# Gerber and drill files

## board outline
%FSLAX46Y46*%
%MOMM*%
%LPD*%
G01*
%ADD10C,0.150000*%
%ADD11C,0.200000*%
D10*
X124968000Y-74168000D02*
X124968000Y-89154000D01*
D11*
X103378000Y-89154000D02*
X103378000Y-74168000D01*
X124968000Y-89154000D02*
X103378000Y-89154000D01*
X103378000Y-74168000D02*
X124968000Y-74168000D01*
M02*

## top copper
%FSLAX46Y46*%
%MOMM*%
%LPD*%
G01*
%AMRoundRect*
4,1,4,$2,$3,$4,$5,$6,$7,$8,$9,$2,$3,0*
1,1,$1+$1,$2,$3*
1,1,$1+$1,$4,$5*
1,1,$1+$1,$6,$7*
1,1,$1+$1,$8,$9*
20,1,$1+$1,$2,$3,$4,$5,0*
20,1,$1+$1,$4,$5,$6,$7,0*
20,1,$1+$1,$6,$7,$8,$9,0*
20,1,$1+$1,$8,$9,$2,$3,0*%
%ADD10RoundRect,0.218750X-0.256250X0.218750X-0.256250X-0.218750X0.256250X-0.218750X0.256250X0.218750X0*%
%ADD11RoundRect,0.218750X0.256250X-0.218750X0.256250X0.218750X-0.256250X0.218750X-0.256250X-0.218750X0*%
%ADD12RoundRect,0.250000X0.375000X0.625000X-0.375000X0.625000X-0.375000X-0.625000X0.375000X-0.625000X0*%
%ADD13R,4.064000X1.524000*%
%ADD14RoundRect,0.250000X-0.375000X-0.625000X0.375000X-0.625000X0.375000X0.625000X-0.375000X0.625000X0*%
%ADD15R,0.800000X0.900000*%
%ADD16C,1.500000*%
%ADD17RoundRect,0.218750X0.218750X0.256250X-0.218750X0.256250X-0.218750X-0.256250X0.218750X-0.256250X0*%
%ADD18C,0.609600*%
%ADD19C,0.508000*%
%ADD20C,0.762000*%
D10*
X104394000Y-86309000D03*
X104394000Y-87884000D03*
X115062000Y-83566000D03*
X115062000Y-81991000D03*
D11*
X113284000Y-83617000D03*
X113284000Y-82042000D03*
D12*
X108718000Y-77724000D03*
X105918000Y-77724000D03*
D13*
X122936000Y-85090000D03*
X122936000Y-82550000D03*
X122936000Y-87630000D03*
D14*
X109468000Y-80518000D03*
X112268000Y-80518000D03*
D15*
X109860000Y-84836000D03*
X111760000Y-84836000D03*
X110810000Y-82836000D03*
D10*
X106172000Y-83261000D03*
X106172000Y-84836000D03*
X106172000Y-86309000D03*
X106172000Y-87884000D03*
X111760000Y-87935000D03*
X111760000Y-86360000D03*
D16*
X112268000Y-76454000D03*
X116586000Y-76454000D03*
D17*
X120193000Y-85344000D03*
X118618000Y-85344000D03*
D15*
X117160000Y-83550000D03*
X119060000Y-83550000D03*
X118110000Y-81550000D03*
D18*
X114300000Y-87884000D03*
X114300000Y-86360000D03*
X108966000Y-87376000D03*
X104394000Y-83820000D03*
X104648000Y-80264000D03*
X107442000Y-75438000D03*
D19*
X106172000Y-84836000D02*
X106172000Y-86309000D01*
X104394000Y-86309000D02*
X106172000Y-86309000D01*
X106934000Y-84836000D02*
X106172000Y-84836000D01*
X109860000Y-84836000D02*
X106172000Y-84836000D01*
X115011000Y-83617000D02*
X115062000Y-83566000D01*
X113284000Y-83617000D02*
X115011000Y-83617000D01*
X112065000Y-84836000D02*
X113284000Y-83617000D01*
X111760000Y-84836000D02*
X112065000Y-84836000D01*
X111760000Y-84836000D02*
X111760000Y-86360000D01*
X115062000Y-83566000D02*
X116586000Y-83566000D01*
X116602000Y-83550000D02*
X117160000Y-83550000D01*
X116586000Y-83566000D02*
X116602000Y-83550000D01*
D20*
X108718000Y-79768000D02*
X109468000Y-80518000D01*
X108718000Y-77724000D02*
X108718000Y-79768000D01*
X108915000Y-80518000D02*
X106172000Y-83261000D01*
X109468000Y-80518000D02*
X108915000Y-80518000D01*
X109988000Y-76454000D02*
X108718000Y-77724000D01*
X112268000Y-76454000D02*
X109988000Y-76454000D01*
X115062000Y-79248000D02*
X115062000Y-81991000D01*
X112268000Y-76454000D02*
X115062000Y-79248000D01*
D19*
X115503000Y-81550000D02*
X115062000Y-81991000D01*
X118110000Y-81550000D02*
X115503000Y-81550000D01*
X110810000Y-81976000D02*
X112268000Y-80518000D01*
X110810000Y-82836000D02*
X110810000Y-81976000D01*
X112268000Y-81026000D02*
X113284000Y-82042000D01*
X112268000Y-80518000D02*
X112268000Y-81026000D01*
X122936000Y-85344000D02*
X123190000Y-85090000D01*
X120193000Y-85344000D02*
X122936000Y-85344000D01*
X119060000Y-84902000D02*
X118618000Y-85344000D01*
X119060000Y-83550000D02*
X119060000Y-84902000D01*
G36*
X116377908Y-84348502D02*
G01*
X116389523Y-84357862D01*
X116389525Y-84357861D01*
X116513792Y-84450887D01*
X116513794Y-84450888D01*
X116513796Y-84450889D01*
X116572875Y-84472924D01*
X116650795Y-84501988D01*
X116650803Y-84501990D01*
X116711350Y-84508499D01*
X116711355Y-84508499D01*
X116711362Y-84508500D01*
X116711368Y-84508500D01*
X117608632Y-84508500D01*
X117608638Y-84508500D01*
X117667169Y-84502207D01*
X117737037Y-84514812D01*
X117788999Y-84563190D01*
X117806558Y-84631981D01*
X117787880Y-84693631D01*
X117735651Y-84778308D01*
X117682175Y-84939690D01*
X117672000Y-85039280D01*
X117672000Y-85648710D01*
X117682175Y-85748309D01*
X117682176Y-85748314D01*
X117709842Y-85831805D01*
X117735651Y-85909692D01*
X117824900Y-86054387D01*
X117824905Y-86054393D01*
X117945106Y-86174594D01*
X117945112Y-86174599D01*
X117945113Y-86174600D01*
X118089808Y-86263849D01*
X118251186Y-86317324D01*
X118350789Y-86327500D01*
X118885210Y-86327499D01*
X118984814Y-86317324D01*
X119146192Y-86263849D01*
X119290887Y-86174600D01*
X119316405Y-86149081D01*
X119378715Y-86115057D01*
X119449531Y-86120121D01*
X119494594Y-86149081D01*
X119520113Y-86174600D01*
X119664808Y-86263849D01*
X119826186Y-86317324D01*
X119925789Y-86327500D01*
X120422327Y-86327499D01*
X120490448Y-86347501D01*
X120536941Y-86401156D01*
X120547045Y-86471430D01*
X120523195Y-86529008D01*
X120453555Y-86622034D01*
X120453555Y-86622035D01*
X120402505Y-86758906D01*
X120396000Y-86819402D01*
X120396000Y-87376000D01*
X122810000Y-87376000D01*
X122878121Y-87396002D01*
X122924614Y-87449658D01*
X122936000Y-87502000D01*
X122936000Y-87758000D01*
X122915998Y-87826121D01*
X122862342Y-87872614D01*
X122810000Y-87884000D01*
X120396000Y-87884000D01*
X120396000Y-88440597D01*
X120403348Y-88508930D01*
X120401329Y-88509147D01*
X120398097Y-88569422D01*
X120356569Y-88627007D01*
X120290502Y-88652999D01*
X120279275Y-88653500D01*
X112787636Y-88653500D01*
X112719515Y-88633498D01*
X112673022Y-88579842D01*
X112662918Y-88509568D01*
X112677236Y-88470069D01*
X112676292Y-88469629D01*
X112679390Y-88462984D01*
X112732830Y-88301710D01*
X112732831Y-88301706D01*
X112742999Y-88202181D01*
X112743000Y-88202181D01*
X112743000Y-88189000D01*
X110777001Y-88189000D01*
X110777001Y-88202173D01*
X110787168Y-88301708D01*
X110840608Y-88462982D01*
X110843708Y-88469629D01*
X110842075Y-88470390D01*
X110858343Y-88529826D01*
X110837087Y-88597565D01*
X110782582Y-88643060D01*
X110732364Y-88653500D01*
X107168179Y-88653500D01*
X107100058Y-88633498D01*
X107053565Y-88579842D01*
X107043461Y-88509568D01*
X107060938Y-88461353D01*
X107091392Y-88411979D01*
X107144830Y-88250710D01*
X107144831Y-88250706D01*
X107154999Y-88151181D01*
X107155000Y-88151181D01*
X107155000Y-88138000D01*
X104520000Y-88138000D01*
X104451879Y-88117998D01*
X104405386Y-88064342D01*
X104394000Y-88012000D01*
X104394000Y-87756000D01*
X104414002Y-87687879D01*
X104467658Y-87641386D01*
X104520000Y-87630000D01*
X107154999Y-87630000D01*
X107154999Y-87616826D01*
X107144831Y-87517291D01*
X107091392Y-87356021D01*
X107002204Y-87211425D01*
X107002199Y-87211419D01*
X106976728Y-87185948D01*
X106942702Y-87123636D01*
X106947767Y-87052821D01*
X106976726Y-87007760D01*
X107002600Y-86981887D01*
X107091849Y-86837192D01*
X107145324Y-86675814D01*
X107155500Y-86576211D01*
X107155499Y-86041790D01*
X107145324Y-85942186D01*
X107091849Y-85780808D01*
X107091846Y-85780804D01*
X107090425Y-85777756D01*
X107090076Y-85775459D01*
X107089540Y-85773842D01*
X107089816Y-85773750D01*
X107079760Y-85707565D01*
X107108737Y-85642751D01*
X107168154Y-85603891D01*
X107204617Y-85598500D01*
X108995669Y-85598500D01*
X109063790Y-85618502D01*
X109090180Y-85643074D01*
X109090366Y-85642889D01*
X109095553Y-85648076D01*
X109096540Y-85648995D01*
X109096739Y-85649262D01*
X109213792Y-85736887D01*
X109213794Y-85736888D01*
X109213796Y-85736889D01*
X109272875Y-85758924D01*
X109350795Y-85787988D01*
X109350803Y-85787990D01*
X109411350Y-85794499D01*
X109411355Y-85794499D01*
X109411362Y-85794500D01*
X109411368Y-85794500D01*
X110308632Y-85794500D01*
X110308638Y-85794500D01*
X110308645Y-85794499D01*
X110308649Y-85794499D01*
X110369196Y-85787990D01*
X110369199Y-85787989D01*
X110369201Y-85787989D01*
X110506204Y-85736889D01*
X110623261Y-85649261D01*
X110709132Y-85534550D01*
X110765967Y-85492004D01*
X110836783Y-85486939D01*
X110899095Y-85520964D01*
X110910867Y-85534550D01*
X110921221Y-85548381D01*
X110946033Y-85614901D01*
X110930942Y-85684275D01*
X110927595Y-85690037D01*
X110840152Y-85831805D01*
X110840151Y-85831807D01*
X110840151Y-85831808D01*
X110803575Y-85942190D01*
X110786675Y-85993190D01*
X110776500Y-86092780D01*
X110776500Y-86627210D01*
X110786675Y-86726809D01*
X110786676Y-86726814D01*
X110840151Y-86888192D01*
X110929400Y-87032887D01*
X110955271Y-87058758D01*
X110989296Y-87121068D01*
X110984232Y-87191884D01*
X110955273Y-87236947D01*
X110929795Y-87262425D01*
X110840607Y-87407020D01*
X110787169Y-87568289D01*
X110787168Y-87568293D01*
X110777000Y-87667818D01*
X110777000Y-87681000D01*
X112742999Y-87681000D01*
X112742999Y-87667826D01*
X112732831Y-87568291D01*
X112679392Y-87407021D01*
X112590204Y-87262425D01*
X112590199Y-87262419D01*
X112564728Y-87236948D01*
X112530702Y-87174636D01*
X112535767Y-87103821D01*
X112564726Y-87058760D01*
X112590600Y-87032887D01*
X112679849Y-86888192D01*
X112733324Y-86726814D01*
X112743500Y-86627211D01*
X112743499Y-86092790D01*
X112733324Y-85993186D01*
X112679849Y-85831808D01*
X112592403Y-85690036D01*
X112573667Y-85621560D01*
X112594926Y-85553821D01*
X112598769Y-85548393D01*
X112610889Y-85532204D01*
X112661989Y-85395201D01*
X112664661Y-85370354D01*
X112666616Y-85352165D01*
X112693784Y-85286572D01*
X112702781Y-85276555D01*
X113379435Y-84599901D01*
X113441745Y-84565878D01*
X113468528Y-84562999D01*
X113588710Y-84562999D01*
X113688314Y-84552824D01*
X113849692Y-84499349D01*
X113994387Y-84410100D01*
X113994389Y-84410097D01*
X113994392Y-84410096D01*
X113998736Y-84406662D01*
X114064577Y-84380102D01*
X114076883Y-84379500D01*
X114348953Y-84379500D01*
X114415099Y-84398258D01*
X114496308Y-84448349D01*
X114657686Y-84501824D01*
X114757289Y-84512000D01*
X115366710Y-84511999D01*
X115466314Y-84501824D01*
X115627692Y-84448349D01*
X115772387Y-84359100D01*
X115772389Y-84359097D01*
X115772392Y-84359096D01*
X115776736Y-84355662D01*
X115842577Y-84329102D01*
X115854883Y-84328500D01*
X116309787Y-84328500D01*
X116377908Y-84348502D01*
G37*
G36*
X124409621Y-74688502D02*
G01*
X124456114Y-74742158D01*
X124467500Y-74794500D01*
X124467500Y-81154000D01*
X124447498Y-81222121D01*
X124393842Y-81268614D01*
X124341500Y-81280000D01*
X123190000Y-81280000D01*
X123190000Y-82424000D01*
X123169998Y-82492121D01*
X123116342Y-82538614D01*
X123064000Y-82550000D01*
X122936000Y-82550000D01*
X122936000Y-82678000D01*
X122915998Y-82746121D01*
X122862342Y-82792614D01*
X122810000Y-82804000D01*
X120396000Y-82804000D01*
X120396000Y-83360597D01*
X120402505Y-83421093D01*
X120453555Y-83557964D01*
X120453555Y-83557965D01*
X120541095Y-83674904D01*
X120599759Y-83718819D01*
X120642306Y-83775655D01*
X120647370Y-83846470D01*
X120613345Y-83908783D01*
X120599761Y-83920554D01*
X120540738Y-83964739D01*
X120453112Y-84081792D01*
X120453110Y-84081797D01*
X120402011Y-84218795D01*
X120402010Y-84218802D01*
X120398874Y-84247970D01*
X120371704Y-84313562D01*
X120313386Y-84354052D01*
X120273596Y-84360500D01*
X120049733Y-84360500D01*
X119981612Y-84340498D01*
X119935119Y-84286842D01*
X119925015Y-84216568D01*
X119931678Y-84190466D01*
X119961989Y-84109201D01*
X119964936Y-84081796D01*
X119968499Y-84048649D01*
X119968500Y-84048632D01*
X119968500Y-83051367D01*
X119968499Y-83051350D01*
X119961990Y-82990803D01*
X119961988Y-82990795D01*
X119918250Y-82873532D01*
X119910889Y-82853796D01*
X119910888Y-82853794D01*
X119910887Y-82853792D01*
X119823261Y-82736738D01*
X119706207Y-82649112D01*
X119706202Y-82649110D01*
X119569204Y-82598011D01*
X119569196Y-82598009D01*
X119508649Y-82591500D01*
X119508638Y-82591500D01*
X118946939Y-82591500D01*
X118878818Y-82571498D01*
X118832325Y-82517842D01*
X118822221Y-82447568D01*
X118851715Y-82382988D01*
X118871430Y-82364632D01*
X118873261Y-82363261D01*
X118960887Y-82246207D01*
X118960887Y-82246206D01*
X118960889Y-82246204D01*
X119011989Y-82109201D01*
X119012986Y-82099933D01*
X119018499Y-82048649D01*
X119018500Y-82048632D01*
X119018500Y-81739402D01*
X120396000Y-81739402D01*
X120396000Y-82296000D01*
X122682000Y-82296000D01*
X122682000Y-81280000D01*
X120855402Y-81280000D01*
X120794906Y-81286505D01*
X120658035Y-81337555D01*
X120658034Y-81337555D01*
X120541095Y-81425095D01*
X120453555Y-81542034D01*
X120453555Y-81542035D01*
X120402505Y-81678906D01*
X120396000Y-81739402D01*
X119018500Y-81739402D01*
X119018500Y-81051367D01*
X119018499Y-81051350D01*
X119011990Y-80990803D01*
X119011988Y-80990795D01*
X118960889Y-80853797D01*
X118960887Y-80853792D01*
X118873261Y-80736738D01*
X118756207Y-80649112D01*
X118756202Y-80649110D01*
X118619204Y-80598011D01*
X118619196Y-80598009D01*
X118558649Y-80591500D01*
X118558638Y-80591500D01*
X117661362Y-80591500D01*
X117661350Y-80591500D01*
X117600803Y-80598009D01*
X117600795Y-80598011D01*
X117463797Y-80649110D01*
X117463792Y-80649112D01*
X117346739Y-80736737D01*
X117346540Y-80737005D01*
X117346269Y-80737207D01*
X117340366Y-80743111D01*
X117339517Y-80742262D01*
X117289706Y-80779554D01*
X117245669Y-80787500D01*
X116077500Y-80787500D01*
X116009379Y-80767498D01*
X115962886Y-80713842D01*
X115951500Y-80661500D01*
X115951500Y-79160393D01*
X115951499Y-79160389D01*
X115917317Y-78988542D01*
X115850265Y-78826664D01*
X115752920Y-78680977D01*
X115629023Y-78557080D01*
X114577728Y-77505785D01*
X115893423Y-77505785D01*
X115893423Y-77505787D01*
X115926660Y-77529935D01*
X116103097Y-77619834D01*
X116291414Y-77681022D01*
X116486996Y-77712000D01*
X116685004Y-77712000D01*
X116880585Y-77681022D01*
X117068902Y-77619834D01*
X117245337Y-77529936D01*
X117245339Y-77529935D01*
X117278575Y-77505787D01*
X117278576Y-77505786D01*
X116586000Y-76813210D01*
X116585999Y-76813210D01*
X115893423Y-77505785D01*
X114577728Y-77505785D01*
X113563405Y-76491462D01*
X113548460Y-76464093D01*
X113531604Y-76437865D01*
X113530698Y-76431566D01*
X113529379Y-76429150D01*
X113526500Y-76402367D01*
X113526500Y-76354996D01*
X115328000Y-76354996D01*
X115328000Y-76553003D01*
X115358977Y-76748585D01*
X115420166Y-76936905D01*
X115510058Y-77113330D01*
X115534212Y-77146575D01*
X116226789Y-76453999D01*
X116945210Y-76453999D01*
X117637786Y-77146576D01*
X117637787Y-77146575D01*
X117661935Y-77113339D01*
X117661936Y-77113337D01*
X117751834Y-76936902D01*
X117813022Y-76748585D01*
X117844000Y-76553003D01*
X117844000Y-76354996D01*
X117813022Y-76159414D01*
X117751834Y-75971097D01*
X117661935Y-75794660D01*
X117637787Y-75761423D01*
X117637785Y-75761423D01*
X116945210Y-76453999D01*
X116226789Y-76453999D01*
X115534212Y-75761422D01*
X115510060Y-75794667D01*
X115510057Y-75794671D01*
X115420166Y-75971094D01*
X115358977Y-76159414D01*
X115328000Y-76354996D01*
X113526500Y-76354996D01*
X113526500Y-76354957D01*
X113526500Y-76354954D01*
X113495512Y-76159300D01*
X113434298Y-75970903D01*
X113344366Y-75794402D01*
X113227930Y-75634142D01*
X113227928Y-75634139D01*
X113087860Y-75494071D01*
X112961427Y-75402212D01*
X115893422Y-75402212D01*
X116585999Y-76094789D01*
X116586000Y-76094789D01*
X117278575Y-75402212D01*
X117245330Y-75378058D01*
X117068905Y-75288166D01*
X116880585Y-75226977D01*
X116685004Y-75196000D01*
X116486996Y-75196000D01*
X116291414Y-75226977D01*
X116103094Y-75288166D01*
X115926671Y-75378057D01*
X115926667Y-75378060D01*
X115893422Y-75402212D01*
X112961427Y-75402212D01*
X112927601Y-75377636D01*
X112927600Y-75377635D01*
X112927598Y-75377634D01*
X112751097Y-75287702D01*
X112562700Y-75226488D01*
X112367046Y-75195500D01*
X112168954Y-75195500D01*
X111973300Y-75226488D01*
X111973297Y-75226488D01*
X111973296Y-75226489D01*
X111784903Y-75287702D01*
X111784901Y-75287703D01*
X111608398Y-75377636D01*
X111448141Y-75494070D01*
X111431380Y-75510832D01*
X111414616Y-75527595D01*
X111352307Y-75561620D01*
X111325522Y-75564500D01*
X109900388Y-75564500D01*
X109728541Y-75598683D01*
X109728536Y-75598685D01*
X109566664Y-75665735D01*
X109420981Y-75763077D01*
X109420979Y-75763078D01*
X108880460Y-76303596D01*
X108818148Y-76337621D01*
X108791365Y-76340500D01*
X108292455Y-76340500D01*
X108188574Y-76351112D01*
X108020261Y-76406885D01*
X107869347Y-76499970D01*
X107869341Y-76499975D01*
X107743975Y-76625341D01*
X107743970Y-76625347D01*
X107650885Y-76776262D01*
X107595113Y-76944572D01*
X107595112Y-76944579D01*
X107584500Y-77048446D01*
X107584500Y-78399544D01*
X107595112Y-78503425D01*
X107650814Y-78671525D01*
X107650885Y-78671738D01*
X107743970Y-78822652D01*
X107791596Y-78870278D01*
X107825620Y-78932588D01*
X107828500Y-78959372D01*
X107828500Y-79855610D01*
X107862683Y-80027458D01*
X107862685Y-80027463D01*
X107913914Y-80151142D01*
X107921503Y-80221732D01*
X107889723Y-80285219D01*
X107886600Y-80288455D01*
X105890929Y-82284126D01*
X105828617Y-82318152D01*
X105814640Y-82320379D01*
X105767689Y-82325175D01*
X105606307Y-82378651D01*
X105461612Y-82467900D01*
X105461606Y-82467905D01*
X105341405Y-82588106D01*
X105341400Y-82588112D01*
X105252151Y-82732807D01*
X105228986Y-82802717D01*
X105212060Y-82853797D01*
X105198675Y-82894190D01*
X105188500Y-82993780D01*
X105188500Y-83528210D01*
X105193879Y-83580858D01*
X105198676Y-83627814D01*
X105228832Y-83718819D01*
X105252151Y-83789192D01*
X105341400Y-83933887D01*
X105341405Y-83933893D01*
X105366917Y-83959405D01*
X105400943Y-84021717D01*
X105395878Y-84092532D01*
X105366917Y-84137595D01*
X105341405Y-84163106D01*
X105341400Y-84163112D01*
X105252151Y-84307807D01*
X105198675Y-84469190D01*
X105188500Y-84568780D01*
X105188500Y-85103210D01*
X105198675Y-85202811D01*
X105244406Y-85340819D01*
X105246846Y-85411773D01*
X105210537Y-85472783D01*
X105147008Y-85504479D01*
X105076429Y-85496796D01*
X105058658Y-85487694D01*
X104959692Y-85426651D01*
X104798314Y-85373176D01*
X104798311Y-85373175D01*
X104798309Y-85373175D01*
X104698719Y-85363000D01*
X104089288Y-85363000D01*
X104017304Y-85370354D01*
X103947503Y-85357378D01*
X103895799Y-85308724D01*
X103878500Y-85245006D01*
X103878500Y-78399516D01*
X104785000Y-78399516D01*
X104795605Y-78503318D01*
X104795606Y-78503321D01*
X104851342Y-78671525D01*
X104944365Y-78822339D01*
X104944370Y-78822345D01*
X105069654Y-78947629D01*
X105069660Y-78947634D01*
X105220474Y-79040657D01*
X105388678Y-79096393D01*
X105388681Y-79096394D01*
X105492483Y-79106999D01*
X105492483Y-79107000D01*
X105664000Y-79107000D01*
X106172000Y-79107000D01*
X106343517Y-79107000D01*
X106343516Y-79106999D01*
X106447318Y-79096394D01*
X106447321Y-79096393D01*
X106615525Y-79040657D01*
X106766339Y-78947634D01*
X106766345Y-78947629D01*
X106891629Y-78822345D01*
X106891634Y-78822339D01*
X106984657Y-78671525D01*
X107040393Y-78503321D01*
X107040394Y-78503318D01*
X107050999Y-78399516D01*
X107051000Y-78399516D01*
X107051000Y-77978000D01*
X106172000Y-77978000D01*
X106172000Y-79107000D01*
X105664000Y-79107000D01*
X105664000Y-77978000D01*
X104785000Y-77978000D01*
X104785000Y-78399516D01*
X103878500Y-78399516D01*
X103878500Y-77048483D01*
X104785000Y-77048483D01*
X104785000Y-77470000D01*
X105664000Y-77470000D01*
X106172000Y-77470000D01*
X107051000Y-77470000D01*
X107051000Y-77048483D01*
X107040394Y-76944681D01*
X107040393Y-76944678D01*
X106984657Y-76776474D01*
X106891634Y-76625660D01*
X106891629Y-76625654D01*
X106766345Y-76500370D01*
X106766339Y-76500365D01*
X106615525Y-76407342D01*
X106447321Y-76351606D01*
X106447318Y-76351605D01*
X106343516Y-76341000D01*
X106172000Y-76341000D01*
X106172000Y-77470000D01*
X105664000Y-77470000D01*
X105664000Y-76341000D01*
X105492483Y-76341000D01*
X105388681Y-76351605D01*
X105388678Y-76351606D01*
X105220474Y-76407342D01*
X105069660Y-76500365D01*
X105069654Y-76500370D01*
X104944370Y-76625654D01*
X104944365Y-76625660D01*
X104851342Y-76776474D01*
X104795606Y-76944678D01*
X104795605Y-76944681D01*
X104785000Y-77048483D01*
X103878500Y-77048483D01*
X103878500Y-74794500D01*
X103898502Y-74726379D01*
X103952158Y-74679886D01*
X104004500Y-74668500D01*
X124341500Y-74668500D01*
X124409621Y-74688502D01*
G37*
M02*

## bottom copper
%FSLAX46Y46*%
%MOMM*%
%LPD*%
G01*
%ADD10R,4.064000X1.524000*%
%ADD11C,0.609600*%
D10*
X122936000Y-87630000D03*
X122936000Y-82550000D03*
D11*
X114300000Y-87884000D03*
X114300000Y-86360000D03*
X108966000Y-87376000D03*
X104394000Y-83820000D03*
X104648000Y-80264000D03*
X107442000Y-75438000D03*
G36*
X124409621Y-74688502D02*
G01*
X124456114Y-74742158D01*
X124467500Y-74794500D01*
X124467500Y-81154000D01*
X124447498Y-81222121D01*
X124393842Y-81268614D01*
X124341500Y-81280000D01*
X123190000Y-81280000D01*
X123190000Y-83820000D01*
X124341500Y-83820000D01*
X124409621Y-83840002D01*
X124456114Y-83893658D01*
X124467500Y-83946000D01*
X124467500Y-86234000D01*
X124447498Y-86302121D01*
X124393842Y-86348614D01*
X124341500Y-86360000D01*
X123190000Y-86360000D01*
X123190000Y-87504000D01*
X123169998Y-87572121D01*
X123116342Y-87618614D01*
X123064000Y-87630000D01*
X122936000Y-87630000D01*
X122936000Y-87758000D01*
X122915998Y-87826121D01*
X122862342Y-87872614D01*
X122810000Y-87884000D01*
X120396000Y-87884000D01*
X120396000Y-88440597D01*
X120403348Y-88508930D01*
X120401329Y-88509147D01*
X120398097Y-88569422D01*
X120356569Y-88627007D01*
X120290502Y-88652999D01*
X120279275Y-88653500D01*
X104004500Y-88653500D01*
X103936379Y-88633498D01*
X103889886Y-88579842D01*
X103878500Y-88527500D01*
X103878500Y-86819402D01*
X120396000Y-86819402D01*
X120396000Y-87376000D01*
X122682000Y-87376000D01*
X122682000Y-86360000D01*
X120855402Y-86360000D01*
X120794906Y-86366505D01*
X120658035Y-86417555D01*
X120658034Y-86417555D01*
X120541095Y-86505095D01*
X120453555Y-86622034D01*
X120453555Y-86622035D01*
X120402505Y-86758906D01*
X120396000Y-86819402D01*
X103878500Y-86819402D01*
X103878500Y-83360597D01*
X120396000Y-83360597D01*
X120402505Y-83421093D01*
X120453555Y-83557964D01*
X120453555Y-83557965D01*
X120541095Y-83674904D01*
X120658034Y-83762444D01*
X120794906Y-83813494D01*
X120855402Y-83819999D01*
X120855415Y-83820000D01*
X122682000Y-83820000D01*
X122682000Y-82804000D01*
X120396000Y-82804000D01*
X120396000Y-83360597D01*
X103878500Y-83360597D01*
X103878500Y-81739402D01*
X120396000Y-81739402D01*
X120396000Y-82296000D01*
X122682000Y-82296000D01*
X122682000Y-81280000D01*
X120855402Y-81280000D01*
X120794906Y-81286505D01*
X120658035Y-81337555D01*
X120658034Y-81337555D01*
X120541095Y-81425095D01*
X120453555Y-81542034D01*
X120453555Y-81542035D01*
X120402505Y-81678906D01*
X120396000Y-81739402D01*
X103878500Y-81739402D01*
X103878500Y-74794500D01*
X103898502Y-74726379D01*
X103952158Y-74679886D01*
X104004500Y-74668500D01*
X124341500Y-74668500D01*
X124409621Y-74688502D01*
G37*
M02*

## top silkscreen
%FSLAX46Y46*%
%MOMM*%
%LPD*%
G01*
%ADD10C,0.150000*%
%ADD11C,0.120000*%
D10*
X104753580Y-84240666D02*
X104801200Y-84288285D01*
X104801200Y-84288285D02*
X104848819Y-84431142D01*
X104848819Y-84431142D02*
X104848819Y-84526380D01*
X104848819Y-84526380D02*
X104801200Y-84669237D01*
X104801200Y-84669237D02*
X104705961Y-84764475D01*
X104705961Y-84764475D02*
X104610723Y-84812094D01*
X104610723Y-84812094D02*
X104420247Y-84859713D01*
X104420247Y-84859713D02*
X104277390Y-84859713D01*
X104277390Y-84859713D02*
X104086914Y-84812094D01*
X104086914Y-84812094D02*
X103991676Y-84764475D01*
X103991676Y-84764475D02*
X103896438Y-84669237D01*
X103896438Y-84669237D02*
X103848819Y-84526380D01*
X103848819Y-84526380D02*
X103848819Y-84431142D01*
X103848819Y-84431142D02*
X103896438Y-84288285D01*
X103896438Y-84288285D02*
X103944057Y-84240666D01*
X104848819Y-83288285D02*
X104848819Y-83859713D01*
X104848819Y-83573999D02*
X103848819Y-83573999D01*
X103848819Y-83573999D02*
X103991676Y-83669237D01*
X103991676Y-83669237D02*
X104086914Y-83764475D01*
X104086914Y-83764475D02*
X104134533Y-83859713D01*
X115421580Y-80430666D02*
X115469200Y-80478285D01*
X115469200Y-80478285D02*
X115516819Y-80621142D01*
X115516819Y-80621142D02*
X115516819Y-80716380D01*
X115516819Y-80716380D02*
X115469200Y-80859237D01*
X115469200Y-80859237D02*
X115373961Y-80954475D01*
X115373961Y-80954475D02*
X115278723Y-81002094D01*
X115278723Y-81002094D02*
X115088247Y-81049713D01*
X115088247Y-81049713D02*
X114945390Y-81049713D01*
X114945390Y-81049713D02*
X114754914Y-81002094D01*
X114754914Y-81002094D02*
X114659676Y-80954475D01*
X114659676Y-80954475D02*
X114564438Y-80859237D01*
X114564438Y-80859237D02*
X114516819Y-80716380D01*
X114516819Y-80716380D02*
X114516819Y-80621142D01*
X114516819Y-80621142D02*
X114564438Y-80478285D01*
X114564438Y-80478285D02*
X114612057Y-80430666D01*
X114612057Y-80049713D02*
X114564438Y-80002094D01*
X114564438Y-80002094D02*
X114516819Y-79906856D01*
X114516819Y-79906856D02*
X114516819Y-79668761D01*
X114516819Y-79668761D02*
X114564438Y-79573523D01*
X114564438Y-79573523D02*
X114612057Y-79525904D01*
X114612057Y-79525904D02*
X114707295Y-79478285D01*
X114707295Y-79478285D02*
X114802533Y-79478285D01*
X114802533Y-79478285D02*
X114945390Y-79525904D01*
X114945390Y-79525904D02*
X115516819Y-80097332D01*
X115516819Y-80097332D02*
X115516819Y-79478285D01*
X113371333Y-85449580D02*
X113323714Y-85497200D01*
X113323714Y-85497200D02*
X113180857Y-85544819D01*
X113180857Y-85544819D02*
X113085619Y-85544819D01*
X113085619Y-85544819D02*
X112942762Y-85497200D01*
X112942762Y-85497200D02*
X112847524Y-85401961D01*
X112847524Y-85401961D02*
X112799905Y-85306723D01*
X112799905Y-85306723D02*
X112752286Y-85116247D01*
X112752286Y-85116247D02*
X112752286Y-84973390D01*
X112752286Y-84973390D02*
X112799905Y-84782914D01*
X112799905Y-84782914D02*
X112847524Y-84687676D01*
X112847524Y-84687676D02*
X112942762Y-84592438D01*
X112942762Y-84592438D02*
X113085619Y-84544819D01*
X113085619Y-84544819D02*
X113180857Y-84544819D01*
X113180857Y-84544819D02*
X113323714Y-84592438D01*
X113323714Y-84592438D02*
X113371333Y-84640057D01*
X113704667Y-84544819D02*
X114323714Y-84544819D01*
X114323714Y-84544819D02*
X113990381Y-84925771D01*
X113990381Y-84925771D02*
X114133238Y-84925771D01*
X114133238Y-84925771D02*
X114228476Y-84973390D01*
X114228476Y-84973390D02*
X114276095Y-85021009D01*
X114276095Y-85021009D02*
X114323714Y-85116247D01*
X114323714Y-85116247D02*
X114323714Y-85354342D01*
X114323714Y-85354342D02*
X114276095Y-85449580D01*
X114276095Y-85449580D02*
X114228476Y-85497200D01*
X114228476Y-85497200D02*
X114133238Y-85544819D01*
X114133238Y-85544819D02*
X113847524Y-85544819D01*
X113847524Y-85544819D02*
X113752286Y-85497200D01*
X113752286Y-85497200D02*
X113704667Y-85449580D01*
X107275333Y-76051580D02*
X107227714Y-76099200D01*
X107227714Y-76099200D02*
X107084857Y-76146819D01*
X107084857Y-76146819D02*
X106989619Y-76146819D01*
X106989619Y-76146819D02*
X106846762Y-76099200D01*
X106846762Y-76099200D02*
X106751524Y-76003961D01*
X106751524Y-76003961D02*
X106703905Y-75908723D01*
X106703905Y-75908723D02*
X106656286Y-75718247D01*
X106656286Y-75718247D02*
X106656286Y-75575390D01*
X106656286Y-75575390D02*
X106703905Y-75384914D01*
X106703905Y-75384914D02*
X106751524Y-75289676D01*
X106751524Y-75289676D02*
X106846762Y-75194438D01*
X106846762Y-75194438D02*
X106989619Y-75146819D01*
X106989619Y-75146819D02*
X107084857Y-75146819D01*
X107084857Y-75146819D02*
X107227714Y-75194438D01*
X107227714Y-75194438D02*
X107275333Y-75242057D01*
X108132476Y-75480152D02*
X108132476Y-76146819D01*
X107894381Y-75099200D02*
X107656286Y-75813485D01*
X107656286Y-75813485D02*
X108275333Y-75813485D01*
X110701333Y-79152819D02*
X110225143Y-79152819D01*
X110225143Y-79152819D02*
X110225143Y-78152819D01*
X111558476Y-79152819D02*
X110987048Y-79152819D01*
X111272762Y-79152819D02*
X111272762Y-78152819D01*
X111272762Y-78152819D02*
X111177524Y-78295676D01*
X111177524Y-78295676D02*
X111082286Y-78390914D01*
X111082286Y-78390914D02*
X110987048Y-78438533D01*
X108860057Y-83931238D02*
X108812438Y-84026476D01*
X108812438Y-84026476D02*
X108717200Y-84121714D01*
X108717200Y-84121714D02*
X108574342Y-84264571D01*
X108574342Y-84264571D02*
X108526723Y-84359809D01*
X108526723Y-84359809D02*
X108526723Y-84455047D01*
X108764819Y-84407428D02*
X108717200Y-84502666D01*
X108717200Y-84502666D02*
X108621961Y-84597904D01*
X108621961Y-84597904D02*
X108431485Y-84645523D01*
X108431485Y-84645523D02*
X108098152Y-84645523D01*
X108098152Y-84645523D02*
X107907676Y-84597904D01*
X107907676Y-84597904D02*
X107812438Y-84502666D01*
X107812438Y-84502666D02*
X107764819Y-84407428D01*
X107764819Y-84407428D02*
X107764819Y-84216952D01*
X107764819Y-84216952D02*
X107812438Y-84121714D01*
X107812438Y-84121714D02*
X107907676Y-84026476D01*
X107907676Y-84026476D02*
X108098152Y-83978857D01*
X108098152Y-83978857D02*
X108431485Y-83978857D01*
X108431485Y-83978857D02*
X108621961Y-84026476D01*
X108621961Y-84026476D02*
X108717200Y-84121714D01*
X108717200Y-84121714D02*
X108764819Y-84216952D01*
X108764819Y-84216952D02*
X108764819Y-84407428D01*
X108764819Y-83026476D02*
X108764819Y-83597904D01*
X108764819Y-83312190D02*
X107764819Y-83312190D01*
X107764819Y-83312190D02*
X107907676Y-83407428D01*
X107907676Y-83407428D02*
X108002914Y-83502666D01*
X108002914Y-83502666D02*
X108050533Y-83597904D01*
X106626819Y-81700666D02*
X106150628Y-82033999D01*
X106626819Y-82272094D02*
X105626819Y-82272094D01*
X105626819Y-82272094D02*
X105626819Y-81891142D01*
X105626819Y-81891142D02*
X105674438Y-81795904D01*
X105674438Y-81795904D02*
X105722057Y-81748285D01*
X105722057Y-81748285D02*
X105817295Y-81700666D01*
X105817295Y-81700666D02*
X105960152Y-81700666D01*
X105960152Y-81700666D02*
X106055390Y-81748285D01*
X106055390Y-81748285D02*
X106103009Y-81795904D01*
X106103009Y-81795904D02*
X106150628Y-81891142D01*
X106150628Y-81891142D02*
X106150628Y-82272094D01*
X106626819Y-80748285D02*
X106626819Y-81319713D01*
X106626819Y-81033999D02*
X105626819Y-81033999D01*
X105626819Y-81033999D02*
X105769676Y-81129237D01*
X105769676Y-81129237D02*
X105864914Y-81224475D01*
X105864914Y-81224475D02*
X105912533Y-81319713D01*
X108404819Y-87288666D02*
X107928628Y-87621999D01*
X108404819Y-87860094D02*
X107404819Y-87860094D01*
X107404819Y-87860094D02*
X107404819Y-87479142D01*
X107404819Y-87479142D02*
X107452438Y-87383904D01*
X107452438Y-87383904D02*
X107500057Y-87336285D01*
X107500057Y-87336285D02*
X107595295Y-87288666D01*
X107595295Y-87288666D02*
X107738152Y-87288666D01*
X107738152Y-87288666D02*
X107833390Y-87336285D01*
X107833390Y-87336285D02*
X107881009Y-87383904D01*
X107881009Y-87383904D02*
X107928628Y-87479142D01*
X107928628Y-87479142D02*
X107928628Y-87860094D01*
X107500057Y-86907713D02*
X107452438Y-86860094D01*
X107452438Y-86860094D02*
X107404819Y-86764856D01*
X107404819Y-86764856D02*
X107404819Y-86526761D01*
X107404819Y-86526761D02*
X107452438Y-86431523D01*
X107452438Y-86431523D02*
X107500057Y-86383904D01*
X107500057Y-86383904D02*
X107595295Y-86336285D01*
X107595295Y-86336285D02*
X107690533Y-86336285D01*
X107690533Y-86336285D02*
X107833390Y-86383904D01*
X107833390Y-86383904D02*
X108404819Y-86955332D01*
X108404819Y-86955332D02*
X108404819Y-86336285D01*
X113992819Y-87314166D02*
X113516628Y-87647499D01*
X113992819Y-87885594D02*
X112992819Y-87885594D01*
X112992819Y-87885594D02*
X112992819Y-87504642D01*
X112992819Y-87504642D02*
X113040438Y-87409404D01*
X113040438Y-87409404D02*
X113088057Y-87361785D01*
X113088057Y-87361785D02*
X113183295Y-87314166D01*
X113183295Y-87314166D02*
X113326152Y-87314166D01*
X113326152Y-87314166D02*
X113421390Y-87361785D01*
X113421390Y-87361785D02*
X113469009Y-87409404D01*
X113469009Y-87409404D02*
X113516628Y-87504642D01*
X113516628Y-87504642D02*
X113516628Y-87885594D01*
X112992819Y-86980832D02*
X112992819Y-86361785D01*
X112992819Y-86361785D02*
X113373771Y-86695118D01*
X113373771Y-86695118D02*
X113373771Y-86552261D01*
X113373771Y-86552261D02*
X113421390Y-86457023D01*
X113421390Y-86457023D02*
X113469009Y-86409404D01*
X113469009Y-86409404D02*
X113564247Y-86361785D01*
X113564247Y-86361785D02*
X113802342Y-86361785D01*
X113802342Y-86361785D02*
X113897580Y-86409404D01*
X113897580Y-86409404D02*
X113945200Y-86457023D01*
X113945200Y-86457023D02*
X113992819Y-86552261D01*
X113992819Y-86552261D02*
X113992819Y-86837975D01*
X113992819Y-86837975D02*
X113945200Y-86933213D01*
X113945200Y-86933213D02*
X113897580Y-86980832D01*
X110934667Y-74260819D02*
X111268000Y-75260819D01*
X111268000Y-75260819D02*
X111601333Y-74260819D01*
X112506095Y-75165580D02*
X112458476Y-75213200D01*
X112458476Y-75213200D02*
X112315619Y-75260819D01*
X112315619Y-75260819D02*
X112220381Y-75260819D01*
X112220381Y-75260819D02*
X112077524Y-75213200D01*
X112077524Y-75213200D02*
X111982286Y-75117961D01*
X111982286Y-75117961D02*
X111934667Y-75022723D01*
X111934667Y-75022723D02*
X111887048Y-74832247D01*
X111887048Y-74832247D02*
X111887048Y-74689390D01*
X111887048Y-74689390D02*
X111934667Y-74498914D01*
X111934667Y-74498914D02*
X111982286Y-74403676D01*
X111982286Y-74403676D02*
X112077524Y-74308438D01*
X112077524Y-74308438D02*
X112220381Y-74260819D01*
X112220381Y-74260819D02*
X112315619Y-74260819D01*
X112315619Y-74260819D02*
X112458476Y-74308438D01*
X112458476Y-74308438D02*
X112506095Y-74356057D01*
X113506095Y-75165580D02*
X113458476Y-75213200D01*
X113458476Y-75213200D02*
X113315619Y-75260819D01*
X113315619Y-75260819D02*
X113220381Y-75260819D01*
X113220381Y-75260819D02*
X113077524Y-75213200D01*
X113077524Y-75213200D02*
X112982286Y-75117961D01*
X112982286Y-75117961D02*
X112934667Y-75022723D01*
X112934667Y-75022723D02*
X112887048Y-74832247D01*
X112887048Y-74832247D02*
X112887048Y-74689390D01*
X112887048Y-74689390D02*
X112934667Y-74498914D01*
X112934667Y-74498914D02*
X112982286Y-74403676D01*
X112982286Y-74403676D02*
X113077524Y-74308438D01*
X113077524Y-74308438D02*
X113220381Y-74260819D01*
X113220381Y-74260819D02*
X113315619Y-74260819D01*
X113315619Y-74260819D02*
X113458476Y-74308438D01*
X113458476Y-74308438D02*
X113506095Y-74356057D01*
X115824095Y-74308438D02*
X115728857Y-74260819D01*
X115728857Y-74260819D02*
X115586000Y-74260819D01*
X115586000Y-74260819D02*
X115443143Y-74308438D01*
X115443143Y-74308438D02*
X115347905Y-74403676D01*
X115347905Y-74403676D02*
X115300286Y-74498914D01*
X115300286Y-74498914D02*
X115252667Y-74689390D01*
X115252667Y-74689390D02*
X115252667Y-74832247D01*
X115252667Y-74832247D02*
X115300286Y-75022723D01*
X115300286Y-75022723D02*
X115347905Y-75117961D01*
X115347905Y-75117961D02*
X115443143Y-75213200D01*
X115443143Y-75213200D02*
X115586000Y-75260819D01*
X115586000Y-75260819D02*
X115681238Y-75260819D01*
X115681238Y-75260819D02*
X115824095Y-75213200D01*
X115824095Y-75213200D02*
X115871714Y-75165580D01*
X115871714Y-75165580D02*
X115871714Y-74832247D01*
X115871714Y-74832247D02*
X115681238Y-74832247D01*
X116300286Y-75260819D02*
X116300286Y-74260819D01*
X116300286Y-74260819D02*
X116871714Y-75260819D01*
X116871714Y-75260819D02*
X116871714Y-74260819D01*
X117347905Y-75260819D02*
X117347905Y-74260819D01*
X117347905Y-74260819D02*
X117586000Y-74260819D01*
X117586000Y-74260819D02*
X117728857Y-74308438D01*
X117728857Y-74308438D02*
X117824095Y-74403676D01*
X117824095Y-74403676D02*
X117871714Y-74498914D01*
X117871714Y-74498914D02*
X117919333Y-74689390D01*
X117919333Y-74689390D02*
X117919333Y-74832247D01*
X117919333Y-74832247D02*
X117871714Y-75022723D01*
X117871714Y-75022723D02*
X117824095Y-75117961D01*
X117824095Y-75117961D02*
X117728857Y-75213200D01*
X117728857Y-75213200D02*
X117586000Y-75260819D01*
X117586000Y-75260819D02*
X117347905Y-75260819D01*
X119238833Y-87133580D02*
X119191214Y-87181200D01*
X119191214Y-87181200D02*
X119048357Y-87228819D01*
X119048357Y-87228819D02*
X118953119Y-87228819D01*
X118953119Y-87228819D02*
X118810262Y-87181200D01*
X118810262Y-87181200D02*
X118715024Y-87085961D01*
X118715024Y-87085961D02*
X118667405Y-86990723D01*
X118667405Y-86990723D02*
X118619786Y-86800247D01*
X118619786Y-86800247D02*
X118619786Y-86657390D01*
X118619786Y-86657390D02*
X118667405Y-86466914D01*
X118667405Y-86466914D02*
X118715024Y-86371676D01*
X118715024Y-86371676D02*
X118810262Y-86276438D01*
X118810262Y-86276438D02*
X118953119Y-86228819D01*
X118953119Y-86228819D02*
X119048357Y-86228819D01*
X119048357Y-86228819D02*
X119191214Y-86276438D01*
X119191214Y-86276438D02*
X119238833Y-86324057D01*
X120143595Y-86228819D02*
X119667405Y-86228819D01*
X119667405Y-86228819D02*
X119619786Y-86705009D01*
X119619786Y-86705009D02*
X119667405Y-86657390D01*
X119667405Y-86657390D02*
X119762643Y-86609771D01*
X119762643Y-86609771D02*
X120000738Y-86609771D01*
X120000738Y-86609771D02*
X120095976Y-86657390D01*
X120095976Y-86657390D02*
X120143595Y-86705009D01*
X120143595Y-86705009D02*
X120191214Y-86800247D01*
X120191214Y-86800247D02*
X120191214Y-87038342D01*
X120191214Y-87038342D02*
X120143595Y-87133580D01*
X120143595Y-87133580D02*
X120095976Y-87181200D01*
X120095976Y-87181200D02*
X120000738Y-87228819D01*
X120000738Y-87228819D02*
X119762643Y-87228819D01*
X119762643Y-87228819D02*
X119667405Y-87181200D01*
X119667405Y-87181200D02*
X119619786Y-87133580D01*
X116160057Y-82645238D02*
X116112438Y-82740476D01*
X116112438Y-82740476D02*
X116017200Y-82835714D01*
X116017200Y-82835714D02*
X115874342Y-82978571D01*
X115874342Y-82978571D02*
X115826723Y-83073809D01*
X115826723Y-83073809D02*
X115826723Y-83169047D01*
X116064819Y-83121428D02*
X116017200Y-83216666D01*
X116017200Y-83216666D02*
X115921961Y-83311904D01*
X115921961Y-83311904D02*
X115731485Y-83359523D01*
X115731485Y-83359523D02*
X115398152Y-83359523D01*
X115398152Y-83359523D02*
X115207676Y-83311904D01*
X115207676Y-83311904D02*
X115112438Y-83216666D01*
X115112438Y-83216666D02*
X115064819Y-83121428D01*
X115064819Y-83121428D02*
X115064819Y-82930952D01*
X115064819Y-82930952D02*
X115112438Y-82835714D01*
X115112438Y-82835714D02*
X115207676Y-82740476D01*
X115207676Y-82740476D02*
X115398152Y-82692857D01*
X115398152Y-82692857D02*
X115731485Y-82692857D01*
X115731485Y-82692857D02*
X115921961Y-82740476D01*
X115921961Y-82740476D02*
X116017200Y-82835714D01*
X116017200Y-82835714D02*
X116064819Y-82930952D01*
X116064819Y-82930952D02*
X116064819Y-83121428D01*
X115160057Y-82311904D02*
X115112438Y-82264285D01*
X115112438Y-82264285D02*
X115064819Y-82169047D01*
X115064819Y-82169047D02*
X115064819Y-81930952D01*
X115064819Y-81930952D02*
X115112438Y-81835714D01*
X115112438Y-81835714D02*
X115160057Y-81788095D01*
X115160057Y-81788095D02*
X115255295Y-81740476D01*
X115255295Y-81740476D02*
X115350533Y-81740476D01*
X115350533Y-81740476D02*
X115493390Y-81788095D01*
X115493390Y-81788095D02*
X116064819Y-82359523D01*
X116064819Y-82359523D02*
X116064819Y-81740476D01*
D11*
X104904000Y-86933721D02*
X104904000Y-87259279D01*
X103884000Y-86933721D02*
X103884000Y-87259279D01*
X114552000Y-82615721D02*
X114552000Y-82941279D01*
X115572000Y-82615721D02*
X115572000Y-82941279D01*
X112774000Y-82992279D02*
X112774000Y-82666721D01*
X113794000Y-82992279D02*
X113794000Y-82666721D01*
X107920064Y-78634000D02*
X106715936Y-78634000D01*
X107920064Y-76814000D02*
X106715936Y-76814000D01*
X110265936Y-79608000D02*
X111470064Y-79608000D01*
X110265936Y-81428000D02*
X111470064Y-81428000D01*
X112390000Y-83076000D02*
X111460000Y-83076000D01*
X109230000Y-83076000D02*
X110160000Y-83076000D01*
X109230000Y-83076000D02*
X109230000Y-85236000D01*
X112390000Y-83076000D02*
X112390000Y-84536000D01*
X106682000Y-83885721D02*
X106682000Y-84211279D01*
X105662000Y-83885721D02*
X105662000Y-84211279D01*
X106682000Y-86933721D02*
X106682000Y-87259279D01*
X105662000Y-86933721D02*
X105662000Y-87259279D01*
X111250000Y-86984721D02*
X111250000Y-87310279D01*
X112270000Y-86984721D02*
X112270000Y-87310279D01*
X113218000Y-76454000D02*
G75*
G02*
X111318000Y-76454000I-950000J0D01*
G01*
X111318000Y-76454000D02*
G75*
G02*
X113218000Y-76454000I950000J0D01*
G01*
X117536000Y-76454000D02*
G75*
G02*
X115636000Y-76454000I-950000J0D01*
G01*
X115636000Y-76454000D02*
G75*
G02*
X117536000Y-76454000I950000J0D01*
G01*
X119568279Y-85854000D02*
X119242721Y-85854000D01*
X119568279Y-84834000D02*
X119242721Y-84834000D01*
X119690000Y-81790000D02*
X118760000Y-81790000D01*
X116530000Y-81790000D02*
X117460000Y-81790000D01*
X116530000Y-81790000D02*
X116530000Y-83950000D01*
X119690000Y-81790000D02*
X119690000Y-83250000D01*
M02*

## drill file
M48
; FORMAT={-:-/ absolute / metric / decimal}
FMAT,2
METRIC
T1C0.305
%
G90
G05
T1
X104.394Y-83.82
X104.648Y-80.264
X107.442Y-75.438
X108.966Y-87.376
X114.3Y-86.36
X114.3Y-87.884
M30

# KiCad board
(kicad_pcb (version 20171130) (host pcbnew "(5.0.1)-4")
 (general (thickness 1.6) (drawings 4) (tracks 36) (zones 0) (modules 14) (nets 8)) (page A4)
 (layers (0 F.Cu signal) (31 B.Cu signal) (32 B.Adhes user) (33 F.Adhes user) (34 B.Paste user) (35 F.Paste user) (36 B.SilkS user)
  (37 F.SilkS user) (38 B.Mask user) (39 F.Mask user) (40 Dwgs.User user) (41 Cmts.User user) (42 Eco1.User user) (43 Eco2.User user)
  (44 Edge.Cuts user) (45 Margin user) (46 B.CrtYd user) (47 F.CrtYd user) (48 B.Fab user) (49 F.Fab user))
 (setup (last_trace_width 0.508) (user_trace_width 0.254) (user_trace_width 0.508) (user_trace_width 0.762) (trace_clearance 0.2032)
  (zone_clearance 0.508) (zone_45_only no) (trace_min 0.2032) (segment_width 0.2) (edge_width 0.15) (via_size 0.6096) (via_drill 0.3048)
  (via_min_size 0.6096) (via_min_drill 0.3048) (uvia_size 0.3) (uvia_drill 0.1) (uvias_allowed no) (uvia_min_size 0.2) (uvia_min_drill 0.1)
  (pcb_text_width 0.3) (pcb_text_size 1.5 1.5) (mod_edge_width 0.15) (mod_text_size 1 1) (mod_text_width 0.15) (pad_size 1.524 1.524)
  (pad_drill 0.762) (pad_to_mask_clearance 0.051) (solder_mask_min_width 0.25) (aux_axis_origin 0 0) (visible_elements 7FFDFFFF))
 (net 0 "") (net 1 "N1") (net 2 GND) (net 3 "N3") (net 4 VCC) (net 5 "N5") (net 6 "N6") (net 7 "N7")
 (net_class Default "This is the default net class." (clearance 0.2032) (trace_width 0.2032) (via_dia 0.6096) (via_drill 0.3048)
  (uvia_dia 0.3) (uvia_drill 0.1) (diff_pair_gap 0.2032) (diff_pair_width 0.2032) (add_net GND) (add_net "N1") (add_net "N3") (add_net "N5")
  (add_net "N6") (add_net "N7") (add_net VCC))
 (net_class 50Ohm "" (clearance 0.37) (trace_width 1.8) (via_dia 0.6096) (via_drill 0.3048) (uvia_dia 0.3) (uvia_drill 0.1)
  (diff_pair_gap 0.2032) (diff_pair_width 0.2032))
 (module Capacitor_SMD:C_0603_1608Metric (layer F.Cu) (at 104.394 87.0965 270)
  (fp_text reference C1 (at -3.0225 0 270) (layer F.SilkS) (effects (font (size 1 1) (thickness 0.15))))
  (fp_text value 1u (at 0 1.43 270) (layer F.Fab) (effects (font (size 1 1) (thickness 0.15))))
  (fp_line (start -0.162779 -0.51) (end 0.162779 -0.51) (layer F.SilkS) (width 0.12))
  (fp_line (start -0.162779 0.51) (end 0.162779 0.51) (layer F.SilkS) (width 0.12))
  (pad 1 smd roundrect (at -0.7875 0 270) (size 0.875 0.95) (layers F.Cu F.Paste F.Mask) (roundrect_rratio 0.25) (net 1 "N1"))
  (pad 2 smd roundrect (at 0.7875 0 270) (size 0.875 0.95) (layers F.Cu F.Paste F.Mask) (roundrect_rratio 0.25) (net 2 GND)))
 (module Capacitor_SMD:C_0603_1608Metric (layer F.Cu) (at 115.062 82.7785 270)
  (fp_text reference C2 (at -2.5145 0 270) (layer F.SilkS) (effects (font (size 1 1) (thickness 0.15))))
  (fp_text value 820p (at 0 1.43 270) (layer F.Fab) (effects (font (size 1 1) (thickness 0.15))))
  (fp_line (start -0.162779 0.51) (end 0.162779 0.51) (layer F.SilkS) (width 0.12))
  (fp_line (start -0.162779 -0.51) (end 0.162779 -0.51) (layer F.SilkS) (width 0.12))
  (pad 2 smd roundrect (at 0.7875 0 270) (size 0.875 0.95) (layers F.Cu F.Paste F.Mask) (roundrect_rratio 0.25) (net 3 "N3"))
  (pad 1 smd roundrect (at -0.7875 0 270) (size 0.875 0.95) (layers F.Cu F.Paste F.Mask) (roundrect_rratio 0.25) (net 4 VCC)))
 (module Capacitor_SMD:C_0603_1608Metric (layer F.Cu) (at 113.284 82.8295 90)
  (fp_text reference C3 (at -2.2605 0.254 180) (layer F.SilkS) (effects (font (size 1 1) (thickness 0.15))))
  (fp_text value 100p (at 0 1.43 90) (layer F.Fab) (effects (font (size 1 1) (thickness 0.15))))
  (fp_line (start -0.162779 -0.51) (end 0.162779 -0.51) (layer F.SilkS) (width 0.12))
  (fp_line (start -0.162779 0.51) (end 0.162779 0.51) (layer F.SilkS) (width 0.12))
  (pad 1 smd roundrect (at -0.7875 0 90) (size 0.875 0.95) (layers F.Cu F.Paste F.Mask) (roundrect_rratio 0.25) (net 3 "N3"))
  (pad 2 smd roundrect (at 0.7875 0 90) (size 0.875 0.95) (layers F.Cu F.Paste F.Mask) (roundrect_rratio 0.25) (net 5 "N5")))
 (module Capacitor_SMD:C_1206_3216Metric (layer F.Cu) (at 107.318 77.724 180)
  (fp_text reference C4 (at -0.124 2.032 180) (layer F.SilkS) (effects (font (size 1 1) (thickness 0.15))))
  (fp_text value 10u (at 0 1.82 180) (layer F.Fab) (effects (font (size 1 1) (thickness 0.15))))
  (fp_line (start -0.602064 -0.91) (end 0.602064 -0.91) (layer F.SilkS) (width 0.12))
  (fp_line (start -0.602064 0.91) (end 0.602064 0.91) (layer F.SilkS) (width 0.12))
  (pad 1 smd roundrect (at -1.4 0 180) (size 1.25 1.75) (layers F.Cu F.Paste F.Mask) (roundrect_rratio 0.2) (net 4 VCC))
  (pad 2 smd roundrect (at 1.4 0 180) (size 1.25 1.75) (layers F.Cu F.Paste F.Mask) (roundrect_rratio 0.2) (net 2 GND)))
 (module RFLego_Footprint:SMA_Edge (layer F.Cu) (at 120.904 85.09)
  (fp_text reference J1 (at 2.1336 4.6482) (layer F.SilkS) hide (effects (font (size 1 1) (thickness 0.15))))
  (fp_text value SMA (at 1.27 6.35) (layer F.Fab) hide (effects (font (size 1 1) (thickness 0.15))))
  (pad 1 smd rect (at 2.032 0) (size 4.064 1.524) (layers F.Cu F.Mask) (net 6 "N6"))
  (pad 2 smd rect (at 2.032 -2.54) (size 4.064 1.524) (layers F.Cu F.Mask) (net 2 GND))
  (pad 2 smd rect (at 2.032 2.54) (size 4.064 1.524) (layers B.Cu B.Mask) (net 2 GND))
  (pad 2 smd rect (at 2.032 -2.54) (size 4.064 1.524) (layers B.Cu B.Mask) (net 2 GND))
  (pad 2 smd rect (at 2.032 2.54) (size 4.064 1.524) (layers F.Cu F.Mask) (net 2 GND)))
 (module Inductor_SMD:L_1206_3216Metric (layer F.Cu) (at 110.868 80.518)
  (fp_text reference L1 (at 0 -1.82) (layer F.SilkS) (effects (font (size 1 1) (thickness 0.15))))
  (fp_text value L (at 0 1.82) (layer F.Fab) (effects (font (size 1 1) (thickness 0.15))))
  (fp_line (start -0.602064 -0.91) (end 0.602064 -0.91) (layer F.SilkS) (width 0.12))
  (fp_line (start -0.602064 0.91) (end 0.602064 0.91) (layer F.SilkS) (width 0.12))
  (pad 1 smd roundrect (at -1.4 0) (size 1.25 1.75) (layers F.Cu F.Paste F.Mask) (roundrect_rratio 0.2) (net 4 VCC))
  (pad 2 smd roundrect (at 1.4 0) (size 1.25 1.75) (layers F.Cu F.Paste F.Mask) (roundrect_rratio 0.2) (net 5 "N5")))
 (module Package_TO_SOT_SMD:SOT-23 (layer F.Cu) (at 110.81 83.836 90)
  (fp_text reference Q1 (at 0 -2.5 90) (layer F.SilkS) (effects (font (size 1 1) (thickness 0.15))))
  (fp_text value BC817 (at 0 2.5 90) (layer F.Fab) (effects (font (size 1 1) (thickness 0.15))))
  (fp_line (start 0.76 1.58) (end 0.76 0.65) (layer F.SilkS) (width 0.12))
  (fp_line (start 0.76 -1.58) (end 0.76 -0.65) (layer F.SilkS) (width 0.12))
  (fp_line (start 0.76 -1.58) (end -1.4 -1.58) (layer F.SilkS) (width 0.12))
  (fp_line (start 0.76 1.58) (end -0.7 1.58) (layer F.SilkS) (width 0.12))
  (pad 1 smd rect (at -1 -0.95 90) (size 0.9 0.8) (layers F.Cu F.Paste F.Mask) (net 1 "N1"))
  (pad 2 smd rect (at -1 0.95 90) (size 0.9 0.8) (layers F.Cu F.Paste F.Mask) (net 3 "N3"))
  (pad 3 smd rect (at 1 0 90) (size 0.9 0.8) (layers F.Cu F.Paste F.Mask) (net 5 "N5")))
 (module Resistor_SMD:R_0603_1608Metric (layer F.Cu) (at 106.172 84.0485 270)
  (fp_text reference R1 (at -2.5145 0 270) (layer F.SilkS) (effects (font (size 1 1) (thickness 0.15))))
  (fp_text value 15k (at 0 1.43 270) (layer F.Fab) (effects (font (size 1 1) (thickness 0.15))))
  (fp_line (start -0.162779 -0.51) (end 0.162779 -0.51) (layer F.SilkS) (width 0.12))
  (fp_line (start -0.162779 0.51) (end 0.162779 0.51) (layer F.SilkS) (width 0.12))
  (pad 1 smd roundrect (at -0.7875 0 270) (size 0.875 0.95) (layers F.Cu F.Paste F.Mask) (roundrect_rratio 0.25) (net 4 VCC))
  (pad 2 smd roundrect (at 0.7875 0 270) (size 0.875 0.95) (layers F.Cu F.Paste F.Mask) (roundrect_rratio 0.25) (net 1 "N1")))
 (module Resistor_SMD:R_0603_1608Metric (layer F.Cu) (at 106.172 87.0965 270)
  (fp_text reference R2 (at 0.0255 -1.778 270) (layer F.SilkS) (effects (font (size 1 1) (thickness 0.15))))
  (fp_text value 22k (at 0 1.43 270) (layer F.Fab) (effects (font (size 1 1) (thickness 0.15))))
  (fp_line (start -0.162779 -0.51) (end 0.162779 -0.51) (layer F.SilkS) (width 0.12))
  (fp_line (start -0.162779 0.51) (end 0.162779 0.51) (layer F.SilkS) (width 0.12))
  (pad 1 smd roundrect (at -0.7875 0 270) (size 0.875 0.95) (layers F.Cu F.Paste F.Mask) (roundrect_rratio 0.25) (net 1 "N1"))
  (pad 2 smd roundrect (at 0.7875 0 270) (size 0.875 0.95) (layers F.Cu F.Paste F.Mask) (roundrect_rratio 0.25) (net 2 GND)))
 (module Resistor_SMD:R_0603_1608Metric (layer F.Cu) (at 111.76 87.1475 270)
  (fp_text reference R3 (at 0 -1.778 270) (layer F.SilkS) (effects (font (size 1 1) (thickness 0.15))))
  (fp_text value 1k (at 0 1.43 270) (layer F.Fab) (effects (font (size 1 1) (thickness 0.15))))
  (fp_line (start -0.162779 0.51) (end 0.162779 0.51) (layer F.SilkS) (width 0.12))
  (fp_line (start -0.162779 -0.51) (end 0.162779 -0.51) (layer F.SilkS) (width 0.12))
  (pad 2 smd roundrect (at 0.7875 0 270) (size 0.875 0.95) (layers F.Cu F.Paste F.Mask) (roundrect_rratio 0.25) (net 2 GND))
  (pad 1 smd roundrect (at -0.7875 0 270) (size 0.875 0.95) (layers F.Cu F.Paste F.Mask) (roundrect_rratio 0.25) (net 3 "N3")))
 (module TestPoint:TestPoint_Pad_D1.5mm (layer F.Cu) (at 112.268 76.454)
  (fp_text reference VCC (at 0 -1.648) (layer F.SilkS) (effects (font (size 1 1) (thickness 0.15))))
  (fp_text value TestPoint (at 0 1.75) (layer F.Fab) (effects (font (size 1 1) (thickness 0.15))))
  (fp_circle (center 0 0) (end 0 0.95) (layer F.SilkS) (width 0.12))
  (pad 1 smd circle (at 0 0) (size 1.5 1.5) (layers F.Cu F.Mask) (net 4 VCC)))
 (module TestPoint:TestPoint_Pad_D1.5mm (layer F.Cu) (at 116.586 76.454)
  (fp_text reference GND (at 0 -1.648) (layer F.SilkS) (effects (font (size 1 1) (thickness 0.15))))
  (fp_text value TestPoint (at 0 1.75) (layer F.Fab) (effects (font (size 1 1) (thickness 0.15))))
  (fp_circle (center 0 0) (end 0 0.95) (layer F.SilkS) (width 0.12))
  (pad 1 smd circle (at 0 0) (size 1.5 1.5) (layers F.Cu F.Mask) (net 2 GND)))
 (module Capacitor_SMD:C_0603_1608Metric (layer F.Cu) (at 119.4055 85.344 180)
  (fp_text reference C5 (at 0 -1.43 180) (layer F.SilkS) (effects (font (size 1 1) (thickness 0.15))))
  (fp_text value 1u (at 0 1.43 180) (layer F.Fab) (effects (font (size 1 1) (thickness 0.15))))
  (fp_line (start -0.162779 -0.51) (end 0.162779 -0.51) (layer F.SilkS) (width 0.12))
  (fp_line (start -0.162779 0.51) (end 0.162779 0.51) (layer F.SilkS) (width 0.12))
  (pad 1 smd roundrect (at -0.7875 0 180) (size 0.875 0.95) (layers F.Cu F.Paste F.Mask) (roundrect_rratio 0.25) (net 6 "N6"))
  (pad 2 smd roundrect (at 0.7875 0 180) (size 0.875 0.95) (layers F.Cu F.Paste F.Mask) (roundrect_rratio 0.25) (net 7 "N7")))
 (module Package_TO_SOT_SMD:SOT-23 (layer F.Cu) (at 118.11 82.55 90)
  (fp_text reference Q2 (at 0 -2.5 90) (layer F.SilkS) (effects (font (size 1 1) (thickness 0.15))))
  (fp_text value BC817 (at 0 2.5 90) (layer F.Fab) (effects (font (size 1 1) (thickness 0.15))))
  (fp_line (start 0.76 1.58) (end 0.76 0.65) (layer F.SilkS) (width 0.12))
  (fp_line (start 0.76 -1.58) (end 0.76 -0.65) (layer F.SilkS) (width 0.12))
  (fp_line (start 0.76 -1.58) (end -1.4 -1.58) (layer F.SilkS) (width 0.12))
  (fp_line (start 0.76 1.58) (end -0.7 1.58) (layer F.SilkS) (width 0.12))
  (pad 1 smd rect (at -1 -0.95 90) (size 0.9 0.8) (layers F.Cu F.Paste F.Mask) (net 3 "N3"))
  (pad 2 smd rect (at -1 0.95 90) (size 0.9 0.8) (layers F.Cu F.Paste F.Mask) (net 7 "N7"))
  (pad 3 smd rect (at 1 0 90) (size 0.9 0.8) (layers F.Cu F.Paste F.Mask) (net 4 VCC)))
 (gr_line (start 124.968 74.168) (end 124.968 89.154) (layer Edge.Cuts) (width 0.15))
 (gr_line (start 103.378 89.154) (end 103.378 74.168) (layer Edge.Cuts) (width 0.2))
 (gr_line (start 124.968 89.154) (end 103.378 89.154) (layer Edge.Cuts) (width 0.2))
 (gr_line (start 103.378 74.168) (end 124.968 74.168) (layer Edge.Cuts) (width 0.2))
 (segment (start 106.172 84.836) (end 106.172 86.309) (width 0.508) (layer F.Cu) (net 1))
 (segment (start 104.394 86.309) (end 106.172 86.309) (width 0.508) (layer F.Cu) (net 1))
 (segment (start 106.934 84.836) (end 106.172 84.836) (width 0.508) (layer F.Cu) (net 1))
 (segment (start 109.86 84.836) (end 106.172 84.836) (width 0.508) (layer F.Cu) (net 1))
 (via (at 114.3 87.884) (size 0.6096) (drill 0.3048) (layers F.Cu B.Cu) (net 2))
 (via (at 114.3 86.36) (size 0.6096) (drill 0.3048) (layers F.Cu B.Cu) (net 2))
 (via (at 108.966 87.376) (size 0.6096) (drill 0.3048) (layers F.Cu B.Cu) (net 2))
 (via (at 104.394 83.82) (size 0.6096) (drill 0.3048) (layers F.Cu B.Cu) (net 2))
 (via (at 104.648 80.264) (size 0.6096) (drill 0.3048) (layers F.Cu B.Cu) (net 2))
 (via (at 107.442 75.438) (size 0.6096) (drill 0.3048) (layers F.Cu B.Cu) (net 2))
 (segment (start 115.011 83.617) (end 115.062 83.566) (width 0.508) (layer F.Cu) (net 3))
 (segment (start 113.284 83.617) (end 115.011 83.617) (width 0.508) (layer F.Cu) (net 3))
 (segment (start 112.065 84.836) (end 113.284 83.617) (width 0.508) (layer F.Cu) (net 3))
 (segment (start 111.76 84.836) (end 112.065 84.836) (width 0.508) (layer F.Cu) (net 3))
 (segment (start 111.76 84.836) (end 111.76 86.36) (width 0.508) (layer F.Cu) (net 3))
 (segment (start 115.062 83.566) (end 116.586 83.566) (width 0.508) (layer F.Cu) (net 3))
 (segment (start 116.602 83.55) (end 117.16 83.55) (width 0.508) (layer F.Cu) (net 3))
 (segment (start 116.586 83.566) (end 116.602 83.55) (width 0.508) (layer F.Cu) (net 3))
 (segment (start 108.718 79.768) (end 109.468 80.518) (width 0.762) (layer F.Cu) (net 4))
 (segment (start 108.718 77.724) (end 108.718 79.768) (width 0.762) (layer F.Cu) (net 4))
 (segment (start 108.915 80.518) (end 106.172 83.261) (width 0.762) (layer F.Cu) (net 4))
 (segment (start 109.468 80.518) (end 108.915 80.518) (width 0.762) (layer F.Cu) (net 4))
 (segment (start 109.988 76.454) (end 108.718 77.724) (width 0.762) (layer F.Cu) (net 4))
 (segment (start 112.268 76.454) (end 109.988 76.454) (width 0.762) (layer F.Cu) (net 4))
 (segment (start 115.062 79.248) (end 115.062 81.991) (width 0.762) (layer F.Cu) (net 4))
 (segment (start 112.268 76.454) (end 115.062 79.248) (width 0.762) (layer F.Cu) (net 4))
 (segment (start 115.503 81.55) (end 115.062 81.991) (width 0.508) (layer F.Cu) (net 4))
 (segment (start 118.11 81.55) (end 115.503 81.55) (width 0.508) (layer F.Cu) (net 4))
 (segment (start 110.81 81.976) (end 112.268 80.518) (width 0.508) (layer F.Cu) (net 5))
 (segment (start 110.81 82.836) (end 110.81 81.976) (width 0.508) (layer F.Cu) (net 5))
 (segment (start 112.268 81.026) (end 113.284 82.042) (width 0.508) (layer F.Cu) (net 5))
 (segment (start 112.268 80.518) (end 112.268 81.026) (width 0.508) (layer F.Cu) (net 5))
 (segment (start 122.936 85.344) (end 123.19 85.09) (width 0.508) (layer F.Cu) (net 6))
 (segment (start 120.193 85.344) (end 122.936 85.344) (width 0.508) (layer F.Cu) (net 6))
 (segment (start 119.06 84.902) (end 118.618 85.344) (width 0.508) (layer F.Cu) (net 7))
 (segment (start 119.06 83.55) (end 119.06 84.902) (width 0.508) (layer F.Cu) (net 7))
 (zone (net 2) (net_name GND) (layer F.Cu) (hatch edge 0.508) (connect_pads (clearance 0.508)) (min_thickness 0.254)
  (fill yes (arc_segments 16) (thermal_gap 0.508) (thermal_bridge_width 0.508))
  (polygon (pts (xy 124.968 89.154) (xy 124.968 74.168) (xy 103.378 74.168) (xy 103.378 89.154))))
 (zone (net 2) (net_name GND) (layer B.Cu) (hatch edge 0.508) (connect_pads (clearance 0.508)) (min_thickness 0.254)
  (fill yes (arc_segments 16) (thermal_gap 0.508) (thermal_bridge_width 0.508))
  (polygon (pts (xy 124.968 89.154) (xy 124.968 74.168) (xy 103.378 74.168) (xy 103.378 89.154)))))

